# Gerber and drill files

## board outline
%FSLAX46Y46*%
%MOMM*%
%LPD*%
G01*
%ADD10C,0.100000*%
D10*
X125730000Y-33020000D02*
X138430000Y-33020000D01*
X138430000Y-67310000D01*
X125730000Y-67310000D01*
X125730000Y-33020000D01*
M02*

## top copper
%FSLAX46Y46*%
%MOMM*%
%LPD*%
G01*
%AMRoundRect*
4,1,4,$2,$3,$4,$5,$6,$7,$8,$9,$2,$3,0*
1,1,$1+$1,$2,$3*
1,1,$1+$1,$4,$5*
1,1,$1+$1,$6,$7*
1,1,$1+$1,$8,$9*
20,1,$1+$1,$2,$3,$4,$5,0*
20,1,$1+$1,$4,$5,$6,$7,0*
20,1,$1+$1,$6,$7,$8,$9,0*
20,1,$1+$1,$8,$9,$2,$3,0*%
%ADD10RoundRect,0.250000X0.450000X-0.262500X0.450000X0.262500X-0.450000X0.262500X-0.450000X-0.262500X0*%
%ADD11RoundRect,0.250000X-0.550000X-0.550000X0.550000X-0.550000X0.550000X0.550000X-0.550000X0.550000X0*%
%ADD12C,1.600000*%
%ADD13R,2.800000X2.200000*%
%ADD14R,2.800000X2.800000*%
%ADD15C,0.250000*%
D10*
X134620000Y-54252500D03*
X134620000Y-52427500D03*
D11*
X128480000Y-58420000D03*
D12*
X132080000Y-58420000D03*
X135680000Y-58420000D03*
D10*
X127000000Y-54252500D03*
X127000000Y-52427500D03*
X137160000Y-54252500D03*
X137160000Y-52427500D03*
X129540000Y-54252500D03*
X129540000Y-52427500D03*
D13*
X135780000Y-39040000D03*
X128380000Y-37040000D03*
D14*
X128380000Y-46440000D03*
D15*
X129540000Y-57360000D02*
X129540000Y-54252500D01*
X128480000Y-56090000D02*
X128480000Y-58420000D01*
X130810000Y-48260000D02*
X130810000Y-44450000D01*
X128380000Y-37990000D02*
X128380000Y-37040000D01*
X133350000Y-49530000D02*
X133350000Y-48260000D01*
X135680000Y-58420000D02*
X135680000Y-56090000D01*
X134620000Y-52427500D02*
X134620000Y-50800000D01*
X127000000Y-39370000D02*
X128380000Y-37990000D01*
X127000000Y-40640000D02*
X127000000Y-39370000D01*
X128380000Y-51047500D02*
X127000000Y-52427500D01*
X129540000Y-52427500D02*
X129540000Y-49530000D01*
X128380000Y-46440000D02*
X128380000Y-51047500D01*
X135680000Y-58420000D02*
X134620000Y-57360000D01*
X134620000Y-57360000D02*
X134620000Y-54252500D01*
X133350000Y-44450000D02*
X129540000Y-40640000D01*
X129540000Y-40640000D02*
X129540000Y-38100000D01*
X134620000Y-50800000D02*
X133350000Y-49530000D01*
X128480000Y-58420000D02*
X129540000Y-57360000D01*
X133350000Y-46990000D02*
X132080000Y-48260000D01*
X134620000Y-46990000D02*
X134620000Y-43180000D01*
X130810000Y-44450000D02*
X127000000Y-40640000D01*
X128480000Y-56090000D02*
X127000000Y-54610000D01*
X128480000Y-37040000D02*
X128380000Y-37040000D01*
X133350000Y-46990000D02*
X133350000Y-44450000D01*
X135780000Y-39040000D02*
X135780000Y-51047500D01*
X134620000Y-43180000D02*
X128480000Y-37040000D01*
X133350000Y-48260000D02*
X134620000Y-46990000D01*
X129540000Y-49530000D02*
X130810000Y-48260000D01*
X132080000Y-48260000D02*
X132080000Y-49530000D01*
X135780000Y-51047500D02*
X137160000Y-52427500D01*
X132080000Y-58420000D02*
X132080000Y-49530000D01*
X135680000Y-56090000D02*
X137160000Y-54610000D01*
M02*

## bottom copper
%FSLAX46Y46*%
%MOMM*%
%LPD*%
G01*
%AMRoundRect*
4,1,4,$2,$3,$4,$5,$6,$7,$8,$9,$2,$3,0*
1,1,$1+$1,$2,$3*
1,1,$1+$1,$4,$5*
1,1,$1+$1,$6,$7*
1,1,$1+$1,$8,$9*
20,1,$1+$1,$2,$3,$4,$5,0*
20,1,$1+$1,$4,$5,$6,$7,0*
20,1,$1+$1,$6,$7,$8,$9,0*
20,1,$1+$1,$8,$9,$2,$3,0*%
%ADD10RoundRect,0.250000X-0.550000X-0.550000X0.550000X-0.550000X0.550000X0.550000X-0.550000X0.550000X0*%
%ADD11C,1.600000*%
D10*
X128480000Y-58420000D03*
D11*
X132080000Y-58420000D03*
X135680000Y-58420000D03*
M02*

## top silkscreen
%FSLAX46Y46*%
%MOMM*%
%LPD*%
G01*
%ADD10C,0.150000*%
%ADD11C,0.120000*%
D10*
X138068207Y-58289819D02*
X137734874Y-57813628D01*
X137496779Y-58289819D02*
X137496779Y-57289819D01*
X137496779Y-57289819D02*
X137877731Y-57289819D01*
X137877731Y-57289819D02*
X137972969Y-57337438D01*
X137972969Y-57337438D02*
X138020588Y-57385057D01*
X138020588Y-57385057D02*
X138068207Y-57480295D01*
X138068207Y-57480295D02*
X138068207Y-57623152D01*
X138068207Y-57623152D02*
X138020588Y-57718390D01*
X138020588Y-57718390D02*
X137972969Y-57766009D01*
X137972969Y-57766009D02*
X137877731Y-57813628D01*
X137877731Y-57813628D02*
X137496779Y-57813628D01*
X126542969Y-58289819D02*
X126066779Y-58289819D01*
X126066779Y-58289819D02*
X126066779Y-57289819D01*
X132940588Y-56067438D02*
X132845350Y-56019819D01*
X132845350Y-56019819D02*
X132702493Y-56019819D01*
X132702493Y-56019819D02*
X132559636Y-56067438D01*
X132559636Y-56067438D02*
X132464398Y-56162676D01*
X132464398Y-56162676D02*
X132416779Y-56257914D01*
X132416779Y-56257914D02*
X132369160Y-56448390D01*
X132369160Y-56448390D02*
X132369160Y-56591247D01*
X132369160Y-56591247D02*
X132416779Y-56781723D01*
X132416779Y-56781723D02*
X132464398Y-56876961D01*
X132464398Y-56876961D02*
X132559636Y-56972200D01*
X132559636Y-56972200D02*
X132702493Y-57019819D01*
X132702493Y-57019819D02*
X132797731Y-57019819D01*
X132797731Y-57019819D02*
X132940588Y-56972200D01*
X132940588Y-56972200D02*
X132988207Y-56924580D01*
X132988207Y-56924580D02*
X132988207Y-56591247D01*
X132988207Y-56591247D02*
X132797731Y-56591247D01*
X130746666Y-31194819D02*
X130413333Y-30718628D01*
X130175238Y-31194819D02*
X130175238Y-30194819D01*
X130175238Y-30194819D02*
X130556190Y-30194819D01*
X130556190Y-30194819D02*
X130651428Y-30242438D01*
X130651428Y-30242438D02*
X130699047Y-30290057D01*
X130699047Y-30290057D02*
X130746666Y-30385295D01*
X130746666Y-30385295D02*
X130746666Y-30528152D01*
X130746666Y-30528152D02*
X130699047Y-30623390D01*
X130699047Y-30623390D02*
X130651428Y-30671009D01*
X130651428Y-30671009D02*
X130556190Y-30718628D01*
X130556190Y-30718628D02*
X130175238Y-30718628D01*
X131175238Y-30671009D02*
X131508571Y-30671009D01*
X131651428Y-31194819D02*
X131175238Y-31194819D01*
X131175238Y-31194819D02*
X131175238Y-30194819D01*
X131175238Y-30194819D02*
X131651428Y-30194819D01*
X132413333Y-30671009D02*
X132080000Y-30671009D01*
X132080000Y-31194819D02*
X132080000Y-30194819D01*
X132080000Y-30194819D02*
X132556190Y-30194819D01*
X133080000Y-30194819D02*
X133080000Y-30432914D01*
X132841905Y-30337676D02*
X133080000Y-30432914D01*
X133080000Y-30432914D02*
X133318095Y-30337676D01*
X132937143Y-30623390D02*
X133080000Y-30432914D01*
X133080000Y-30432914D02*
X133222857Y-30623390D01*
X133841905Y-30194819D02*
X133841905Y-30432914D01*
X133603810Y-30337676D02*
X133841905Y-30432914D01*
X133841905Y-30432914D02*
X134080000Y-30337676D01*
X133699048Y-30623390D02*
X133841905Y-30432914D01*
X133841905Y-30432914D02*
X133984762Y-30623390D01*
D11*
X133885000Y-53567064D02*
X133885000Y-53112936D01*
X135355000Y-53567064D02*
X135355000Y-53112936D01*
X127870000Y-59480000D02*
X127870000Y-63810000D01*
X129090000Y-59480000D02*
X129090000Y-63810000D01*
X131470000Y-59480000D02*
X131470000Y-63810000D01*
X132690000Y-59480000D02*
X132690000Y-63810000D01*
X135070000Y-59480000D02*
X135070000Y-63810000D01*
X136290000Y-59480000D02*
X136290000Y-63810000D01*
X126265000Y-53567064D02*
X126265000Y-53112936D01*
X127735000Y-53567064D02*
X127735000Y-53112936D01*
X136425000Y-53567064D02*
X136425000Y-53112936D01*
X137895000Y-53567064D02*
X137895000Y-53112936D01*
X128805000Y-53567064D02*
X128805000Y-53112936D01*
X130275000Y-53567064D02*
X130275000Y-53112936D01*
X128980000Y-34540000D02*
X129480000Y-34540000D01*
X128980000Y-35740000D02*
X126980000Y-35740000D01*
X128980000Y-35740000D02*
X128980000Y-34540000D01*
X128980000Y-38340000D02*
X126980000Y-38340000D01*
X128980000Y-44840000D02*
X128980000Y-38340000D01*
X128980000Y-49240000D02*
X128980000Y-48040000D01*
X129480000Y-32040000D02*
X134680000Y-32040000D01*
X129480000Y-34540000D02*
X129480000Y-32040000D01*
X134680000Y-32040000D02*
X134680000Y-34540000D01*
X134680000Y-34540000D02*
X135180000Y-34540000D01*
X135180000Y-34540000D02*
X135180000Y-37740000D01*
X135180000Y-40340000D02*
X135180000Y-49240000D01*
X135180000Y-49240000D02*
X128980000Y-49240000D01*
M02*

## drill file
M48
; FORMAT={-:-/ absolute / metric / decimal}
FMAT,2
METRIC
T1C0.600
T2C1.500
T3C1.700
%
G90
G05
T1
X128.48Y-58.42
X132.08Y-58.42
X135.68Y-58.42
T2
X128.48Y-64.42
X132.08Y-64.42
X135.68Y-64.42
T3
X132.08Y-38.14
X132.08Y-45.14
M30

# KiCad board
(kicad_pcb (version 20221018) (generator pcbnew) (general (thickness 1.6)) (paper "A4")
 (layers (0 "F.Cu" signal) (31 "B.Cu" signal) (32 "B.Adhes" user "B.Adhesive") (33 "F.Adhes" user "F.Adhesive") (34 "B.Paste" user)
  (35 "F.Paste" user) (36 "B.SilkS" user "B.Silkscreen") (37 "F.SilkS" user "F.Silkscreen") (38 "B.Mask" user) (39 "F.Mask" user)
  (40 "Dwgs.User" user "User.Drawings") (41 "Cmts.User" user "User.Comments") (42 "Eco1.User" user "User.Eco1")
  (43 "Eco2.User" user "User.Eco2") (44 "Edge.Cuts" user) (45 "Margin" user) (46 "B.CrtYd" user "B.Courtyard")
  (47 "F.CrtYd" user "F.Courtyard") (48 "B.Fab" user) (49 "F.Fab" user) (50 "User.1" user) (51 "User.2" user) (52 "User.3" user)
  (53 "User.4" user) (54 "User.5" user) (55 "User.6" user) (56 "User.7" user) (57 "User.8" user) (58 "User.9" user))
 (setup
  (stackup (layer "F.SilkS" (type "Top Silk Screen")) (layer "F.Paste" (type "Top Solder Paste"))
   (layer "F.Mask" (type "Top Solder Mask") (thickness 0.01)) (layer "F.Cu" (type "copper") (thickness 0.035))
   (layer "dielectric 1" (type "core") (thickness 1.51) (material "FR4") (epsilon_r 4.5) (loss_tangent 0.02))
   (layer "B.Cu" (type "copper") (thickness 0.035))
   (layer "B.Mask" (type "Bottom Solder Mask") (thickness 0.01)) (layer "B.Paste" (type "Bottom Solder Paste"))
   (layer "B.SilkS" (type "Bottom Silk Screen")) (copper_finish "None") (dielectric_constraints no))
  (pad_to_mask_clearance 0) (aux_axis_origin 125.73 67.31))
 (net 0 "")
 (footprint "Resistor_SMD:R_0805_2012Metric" (layer "F.Cu") (at 134.62 53.34 90)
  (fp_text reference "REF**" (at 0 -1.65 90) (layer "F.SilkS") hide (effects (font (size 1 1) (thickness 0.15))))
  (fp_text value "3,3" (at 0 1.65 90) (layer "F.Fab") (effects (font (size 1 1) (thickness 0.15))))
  (fp_line (start -0.227064 -0.735) (end 0.227064 -0.735) (stroke (width 0.12) (type solid)) (layer "F.SilkS"))
  (fp_line (start -0.227064 0.735) (end 0.227064 0.735) (stroke (width 0.12) (type solid)) (layer "F.SilkS"))
  (pad "1" smd roundrect (at -0.9125 0 90) (size 1.025 1.4) (layers "F.Cu" "F.Paste" "F.Mask") (roundrect_rratio 0.243902439))
  (pad "2" smd roundrect (at 0.9125 0 90) (size 1.025 1.4) (layers "F.Cu" "F.Paste" "F.Mask") (roundrect_rratio 0.243902439)))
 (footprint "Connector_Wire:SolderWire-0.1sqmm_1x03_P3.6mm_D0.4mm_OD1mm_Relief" (layer "F.Cu") (at 128.48 58.42)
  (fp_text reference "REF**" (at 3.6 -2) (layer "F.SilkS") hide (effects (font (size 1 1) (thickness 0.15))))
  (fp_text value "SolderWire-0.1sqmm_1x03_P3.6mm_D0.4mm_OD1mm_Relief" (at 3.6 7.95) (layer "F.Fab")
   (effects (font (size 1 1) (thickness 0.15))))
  (fp_line (start -0.61 1.06) (end -0.61 5.39) (stroke (width 0.12) (type solid)) (layer "F.SilkS"))
  (fp_line (start 0.61 1.06) (end 0.61 5.39) (stroke (width 0.12) (type solid)) (layer "F.SilkS"))
  (fp_line (start 2.99 1.06) (end 2.99 5.39) (stroke (width 0.12) (type solid)) (layer "F.SilkS"))
  (fp_line (start 4.21 1.06) (end 4.21 5.39) (stroke (width 0.12) (type solid)) (layer "F.SilkS"))
  (fp_line (start 6.59 1.06) (end 6.59 5.39) (stroke (width 0.12) (type solid)) (layer "F.SilkS"))
  (fp_line (start 7.81 1.06) (end 7.81 5.39) (stroke (width 0.12) (type solid)) (layer "F.SilkS"))
  (pad "" np_thru_hole circle (at 0 6) (size 1.5 1.5) (drill 1.5) (layers "*.Cu" "*.Mask"))
  (pad "" np_thru_hole circle (at 3.6 6) (size 1.5 1.5) (drill 1.5) (layers "*.Cu" "*.Mask"))
  (pad "" np_thru_hole circle (at 7.2 6) (size 1.5 1.5) (drill 1.5) (layers "*.Cu" "*.Mask"))
  (pad "1" thru_hole roundrect (at 0 0) (size 1.6 1.6) (drill 0.6) (layers "*.Cu" "*.Mask") (roundrect_rratio 0.15625))
  (pad "2" thru_hole circle (at 3.6 0) (size 1.6 1.6) (drill 0.6) (layers "*.Cu" "*.Mask"))
  (pad "3" thru_hole circle (at 7.2 0) (size 1.6 1.6) (drill 0.6) (layers "*.Cu" "*.Mask")))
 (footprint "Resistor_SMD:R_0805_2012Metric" (layer "F.Cu") (at 127 53.34 90)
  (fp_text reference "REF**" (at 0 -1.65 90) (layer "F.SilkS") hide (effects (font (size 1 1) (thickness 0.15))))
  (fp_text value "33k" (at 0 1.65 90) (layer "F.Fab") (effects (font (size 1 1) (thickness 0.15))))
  (fp_line (start -0.227064 -0.735) (end 0.227064 -0.735) (stroke (width 0.12) (type solid)) (layer "F.SilkS"))
  (fp_line (start -0.227064 0.735) (end 0.227064 0.735) (stroke (width 0.12) (type solid)) (layer "F.SilkS"))
  (pad "1" smd roundrect (at -0.9125 0 90) (size 1.025 1.4) (layers "F.Cu" "F.Paste" "F.Mask") (roundrect_rratio 0.243902439))
  (pad "2" smd roundrect (at 0.9125 0 90) (size 1.025 1.4) (layers "F.Cu" "F.Paste" "F.Mask") (roundrect_rratio 0.243902439)))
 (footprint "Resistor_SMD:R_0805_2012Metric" (layer "F.Cu") (at 137.16 53.34 90)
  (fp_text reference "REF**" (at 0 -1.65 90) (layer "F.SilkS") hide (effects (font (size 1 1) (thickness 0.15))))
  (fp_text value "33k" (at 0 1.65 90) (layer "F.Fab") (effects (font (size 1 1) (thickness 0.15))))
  (fp_line (start -0.227064 -0.735) (end 0.227064 -0.735) (stroke (width 0.12) (type solid)) (layer "F.SilkS"))
  (fp_line (start -0.227064 0.735) (end 0.227064 0.735) (stroke (width 0.12) (type solid)) (layer "F.SilkS"))
  (pad "1" smd roundrect (at -0.9125 0 90) (size 1.025 1.4) (layers "F.Cu" "F.Paste" "F.Mask") (roundrect_rratio 0.243902439))
  (pad "2" smd roundrect (at 0.9125 0 90) (size 1.025 1.4) (layers "F.Cu" "F.Paste" "F.Mask") (roundrect_rratio 0.243902439)))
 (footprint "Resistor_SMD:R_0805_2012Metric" (layer "F.Cu") (at 129.54 53.34 90)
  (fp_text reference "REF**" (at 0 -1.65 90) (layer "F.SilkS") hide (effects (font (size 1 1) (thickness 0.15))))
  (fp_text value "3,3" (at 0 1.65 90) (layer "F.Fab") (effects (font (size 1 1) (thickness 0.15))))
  (fp_line (start -0.227064 -0.735) (end 0.227064 -0.735) (stroke (width 0.12) (type solid)) (layer "F.SilkS"))
  (fp_line (start -0.227064 0.735) (end 0.227064 0.735) (stroke (width 0.12) (type solid)) (layer "F.SilkS"))
  (pad "1" smd roundrect (at -0.9125 0 90) (size 1.025 1.4) (layers "F.Cu" "F.Paste" "F.Mask") (roundrect_rratio 0.243902439))
  (pad "2" smd roundrect (at 0.9125 0 90) (size 1.025 1.4) (layers "F.Cu" "F.Paste" "F.Mask") (roundrect_rratio 0.243902439)))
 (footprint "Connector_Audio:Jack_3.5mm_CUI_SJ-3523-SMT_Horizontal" (layer "F.Cu") (at 132.08 40.64)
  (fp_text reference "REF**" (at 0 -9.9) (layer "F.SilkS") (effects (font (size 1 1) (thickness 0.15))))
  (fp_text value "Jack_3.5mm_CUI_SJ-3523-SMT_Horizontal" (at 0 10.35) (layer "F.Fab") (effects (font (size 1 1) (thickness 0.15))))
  (fp_line (start -3.1 -6.1) (end -2.6 -6.1) (stroke (width 0.12) (type solid)) (layer "F.SilkS"))
  (fp_line (start -3.1 -4.9) (end -5.1 -4.9) (stroke (width 0.12) (type solid)) (layer "F.SilkS"))
  (fp_line (start -3.1 -4.9) (end -3.1 -6.1) (stroke (width 0.12) (type solid)) (layer "F.SilkS"))
  (fp_line (start -3.1 -2.3) (end -5.1 -2.3) (stroke (width 0.12) (type solid)) (layer "F.SilkS"))
  (fp_line (start -3.1 4.2) (end -3.1 -2.3) (stroke (width 0.12) (type solid)) (layer "F.SilkS"))
  (fp_line (start -3.1 8.6) (end -3.1 7.4) (stroke (width 0.12) (type solid)) (layer "F.SilkS"))
  (fp_line (start -2.6 -8.6) (end 2.6 -8.6) (stroke (width 0.12) (type solid)) (layer "F.SilkS"))
  (fp_line (start -2.6 -6.1) (end -2.6 -8.6) (stroke (width 0.12) (type solid)) (layer "F.SilkS"))
  (fp_line (start 2.6 -8.6) (end 2.6 -6.1) (stroke (width 0.12) (type solid)) (layer "F.SilkS"))
  (fp_line (start 2.6 -6.1) (end 3.1 -6.1) (stroke (width 0.12) (type solid)) (layer "F.SilkS"))
  (fp_line (start 3.1 -6.1) (end 3.1 -2.9) (stroke (width 0.12) (type solid)) (layer "F.SilkS"))
  (fp_line (start 3.1 -0.3) (end 3.1 8.6) (stroke (width 0.12) (type solid)) (layer "F.SilkS"))
  (fp_line (start 3.1 8.6) (end -3.1 8.6) (stroke (width 0.12) (type solid)) (layer "F.SilkS"))
  (pad "" np_thru_hole circle (at 0 -2.5) (size 1.7 1.7) (drill 1.7) (layers "*.Cu" "*.Mask"))
  (pad "" np_thru_hole circle (at 0 4.5) (size 1.7 1.7) (drill 1.7) (layers "*.Cu" "*.Mask"))
  (pad "R" smd rect (at 3.7 -1.6) (size 2.8 2.2) (layers "F.Cu" "F.Paste" "F.Mask"))
  (pad "S" smd rect (at -3.7 -3.6) (size 2.8 2.2) (layers "F.Cu" "F.Paste" "F.Mask"))
  (pad "T" smd rect (at -3.7 5.8) (size 2.8 2.8) (layers "F.Cu" "F.Paste" "F.Mask")))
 (gr_poly
  (pts (xy 125.73 33.02) (xy 138.43 33.02) (xy 138.43 67.31) (xy 125.73 67.31)) (stroke (width 0.1) (type solid)) (fill none)
  (layer "Edge.Cuts"))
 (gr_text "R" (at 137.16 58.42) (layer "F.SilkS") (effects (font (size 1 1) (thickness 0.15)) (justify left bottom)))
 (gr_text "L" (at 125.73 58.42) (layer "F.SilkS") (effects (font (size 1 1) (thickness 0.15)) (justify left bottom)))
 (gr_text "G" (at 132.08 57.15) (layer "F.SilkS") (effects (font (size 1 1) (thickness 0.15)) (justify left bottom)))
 (segment (start 129.54 57.36) (end 129.54 54.2525) (width 0.25) (layer "F.Cu") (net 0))
 (segment (start 128.48 56.09) (end 128.48 58.42) (width 0.25) (layer "F.Cu") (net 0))
 (segment (start 130.81 48.26) (end 130.81 44.45) (width 0.25) (layer "F.Cu") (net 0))
 (segment (start 128.38 37.99) (end 128.38 37.04) (width 0.25) (layer "F.Cu") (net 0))
 (segment (start 133.35 49.53) (end 133.35 48.26) (width 0.25) (layer "F.Cu") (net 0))
 (segment (start 135.68 58.42) (end 135.68 56.09) (width 0.25) (layer "F.Cu") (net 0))
 (segment (start 134.62 52.4275) (end 134.62 50.8) (width 0.25) (layer "F.Cu") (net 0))
 (segment (start 127 39.37) (end 128.38 37.99) (width 0.25) (layer "F.Cu") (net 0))
 (segment (start 127 40.64) (end 127 39.37) (width 0.25) (layer "F.Cu") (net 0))
 (segment (start 128.38 51.0475) (end 127 52.4275) (width 0.25) (layer "F.Cu") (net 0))
 (segment (start 129.54 52.4275) (end 129.54 49.53) (width 0.25) (layer "F.Cu") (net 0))
 (segment (start 128.38 46.44) (end 128.38 51.0475) (width 0.25) (layer "F.Cu") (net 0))
 (segment (start 135.68 58.42) (end 134.62 57.36) (width 0.25) (layer "F.Cu") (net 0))
 (segment (start 134.62 57.36) (end 134.62 54.2525) (width 0.25) (layer "F.Cu") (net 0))
 (segment (start 133.35 44.45) (end 129.54 40.64) (width 0.25) (layer "F.Cu") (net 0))
 (segment (start 129.54 40.64) (end 129.54 38.1) (width 0.25) (layer "F.Cu") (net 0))
 (segment (start 134.62 50.8) (end 133.35 49.53) (width 0.25) (layer "F.Cu") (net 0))
 (segment (start 128.48 58.42) (end 129.54 57.36) (width 0.25) (layer "F.Cu") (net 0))
 (segment (start 133.35 46.99) (end 132.08 48.26) (width 0.25) (layer "F.Cu") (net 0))
 (segment (start 134.62 46.99) (end 134.62 43.18) (width 0.25) (layer "F.Cu") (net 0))
 (segment (start 130.81 44.45) (end 127 40.64) (width 0.25) (layer "F.Cu") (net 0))
 (segment (start 128.48 56.09) (end 127 54.61) (width 0.25) (layer "F.Cu") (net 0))
 (segment (start 128.48 37.04) (end 128.38 37.04) (width 0.25) (layer "F.Cu") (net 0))
 (segment (start 133.35 46.99) (end 133.35 44.45) (width 0.25) (layer "F.Cu") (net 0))
 (segment (start 135.78 39.04) (end 135.78 51.0475) (width 0.25) (layer "F.Cu") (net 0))
 (segment (start 134.62 43.18) (end 128.48 37.04) (width 0.25) (layer "F.Cu") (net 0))
 (segment (start 133.35 48.26) (end 134.62 46.99) (width 0.25) (layer "F.Cu") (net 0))
 (segment (start 129.54 49.53) (end 130.81 48.26) (width 0.25) (layer "F.Cu") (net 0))
 (segment (start 132.08 48.26) (end 132.08 49.53) (width 0.25) (layer "F.Cu") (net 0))
 (segment (start 135.78 51.0475) (end 137.16 52.4275) (width 0.25) (layer "F.Cu") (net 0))
 (segment (start 132.08 58.42) (end 132.08 49.53) (width 0.25) (layer "F.Cu") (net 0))
 (segment (start 135.68 56.09) (end 137.16 54.61) (width 0.25) (layer "F.Cu") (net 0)))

